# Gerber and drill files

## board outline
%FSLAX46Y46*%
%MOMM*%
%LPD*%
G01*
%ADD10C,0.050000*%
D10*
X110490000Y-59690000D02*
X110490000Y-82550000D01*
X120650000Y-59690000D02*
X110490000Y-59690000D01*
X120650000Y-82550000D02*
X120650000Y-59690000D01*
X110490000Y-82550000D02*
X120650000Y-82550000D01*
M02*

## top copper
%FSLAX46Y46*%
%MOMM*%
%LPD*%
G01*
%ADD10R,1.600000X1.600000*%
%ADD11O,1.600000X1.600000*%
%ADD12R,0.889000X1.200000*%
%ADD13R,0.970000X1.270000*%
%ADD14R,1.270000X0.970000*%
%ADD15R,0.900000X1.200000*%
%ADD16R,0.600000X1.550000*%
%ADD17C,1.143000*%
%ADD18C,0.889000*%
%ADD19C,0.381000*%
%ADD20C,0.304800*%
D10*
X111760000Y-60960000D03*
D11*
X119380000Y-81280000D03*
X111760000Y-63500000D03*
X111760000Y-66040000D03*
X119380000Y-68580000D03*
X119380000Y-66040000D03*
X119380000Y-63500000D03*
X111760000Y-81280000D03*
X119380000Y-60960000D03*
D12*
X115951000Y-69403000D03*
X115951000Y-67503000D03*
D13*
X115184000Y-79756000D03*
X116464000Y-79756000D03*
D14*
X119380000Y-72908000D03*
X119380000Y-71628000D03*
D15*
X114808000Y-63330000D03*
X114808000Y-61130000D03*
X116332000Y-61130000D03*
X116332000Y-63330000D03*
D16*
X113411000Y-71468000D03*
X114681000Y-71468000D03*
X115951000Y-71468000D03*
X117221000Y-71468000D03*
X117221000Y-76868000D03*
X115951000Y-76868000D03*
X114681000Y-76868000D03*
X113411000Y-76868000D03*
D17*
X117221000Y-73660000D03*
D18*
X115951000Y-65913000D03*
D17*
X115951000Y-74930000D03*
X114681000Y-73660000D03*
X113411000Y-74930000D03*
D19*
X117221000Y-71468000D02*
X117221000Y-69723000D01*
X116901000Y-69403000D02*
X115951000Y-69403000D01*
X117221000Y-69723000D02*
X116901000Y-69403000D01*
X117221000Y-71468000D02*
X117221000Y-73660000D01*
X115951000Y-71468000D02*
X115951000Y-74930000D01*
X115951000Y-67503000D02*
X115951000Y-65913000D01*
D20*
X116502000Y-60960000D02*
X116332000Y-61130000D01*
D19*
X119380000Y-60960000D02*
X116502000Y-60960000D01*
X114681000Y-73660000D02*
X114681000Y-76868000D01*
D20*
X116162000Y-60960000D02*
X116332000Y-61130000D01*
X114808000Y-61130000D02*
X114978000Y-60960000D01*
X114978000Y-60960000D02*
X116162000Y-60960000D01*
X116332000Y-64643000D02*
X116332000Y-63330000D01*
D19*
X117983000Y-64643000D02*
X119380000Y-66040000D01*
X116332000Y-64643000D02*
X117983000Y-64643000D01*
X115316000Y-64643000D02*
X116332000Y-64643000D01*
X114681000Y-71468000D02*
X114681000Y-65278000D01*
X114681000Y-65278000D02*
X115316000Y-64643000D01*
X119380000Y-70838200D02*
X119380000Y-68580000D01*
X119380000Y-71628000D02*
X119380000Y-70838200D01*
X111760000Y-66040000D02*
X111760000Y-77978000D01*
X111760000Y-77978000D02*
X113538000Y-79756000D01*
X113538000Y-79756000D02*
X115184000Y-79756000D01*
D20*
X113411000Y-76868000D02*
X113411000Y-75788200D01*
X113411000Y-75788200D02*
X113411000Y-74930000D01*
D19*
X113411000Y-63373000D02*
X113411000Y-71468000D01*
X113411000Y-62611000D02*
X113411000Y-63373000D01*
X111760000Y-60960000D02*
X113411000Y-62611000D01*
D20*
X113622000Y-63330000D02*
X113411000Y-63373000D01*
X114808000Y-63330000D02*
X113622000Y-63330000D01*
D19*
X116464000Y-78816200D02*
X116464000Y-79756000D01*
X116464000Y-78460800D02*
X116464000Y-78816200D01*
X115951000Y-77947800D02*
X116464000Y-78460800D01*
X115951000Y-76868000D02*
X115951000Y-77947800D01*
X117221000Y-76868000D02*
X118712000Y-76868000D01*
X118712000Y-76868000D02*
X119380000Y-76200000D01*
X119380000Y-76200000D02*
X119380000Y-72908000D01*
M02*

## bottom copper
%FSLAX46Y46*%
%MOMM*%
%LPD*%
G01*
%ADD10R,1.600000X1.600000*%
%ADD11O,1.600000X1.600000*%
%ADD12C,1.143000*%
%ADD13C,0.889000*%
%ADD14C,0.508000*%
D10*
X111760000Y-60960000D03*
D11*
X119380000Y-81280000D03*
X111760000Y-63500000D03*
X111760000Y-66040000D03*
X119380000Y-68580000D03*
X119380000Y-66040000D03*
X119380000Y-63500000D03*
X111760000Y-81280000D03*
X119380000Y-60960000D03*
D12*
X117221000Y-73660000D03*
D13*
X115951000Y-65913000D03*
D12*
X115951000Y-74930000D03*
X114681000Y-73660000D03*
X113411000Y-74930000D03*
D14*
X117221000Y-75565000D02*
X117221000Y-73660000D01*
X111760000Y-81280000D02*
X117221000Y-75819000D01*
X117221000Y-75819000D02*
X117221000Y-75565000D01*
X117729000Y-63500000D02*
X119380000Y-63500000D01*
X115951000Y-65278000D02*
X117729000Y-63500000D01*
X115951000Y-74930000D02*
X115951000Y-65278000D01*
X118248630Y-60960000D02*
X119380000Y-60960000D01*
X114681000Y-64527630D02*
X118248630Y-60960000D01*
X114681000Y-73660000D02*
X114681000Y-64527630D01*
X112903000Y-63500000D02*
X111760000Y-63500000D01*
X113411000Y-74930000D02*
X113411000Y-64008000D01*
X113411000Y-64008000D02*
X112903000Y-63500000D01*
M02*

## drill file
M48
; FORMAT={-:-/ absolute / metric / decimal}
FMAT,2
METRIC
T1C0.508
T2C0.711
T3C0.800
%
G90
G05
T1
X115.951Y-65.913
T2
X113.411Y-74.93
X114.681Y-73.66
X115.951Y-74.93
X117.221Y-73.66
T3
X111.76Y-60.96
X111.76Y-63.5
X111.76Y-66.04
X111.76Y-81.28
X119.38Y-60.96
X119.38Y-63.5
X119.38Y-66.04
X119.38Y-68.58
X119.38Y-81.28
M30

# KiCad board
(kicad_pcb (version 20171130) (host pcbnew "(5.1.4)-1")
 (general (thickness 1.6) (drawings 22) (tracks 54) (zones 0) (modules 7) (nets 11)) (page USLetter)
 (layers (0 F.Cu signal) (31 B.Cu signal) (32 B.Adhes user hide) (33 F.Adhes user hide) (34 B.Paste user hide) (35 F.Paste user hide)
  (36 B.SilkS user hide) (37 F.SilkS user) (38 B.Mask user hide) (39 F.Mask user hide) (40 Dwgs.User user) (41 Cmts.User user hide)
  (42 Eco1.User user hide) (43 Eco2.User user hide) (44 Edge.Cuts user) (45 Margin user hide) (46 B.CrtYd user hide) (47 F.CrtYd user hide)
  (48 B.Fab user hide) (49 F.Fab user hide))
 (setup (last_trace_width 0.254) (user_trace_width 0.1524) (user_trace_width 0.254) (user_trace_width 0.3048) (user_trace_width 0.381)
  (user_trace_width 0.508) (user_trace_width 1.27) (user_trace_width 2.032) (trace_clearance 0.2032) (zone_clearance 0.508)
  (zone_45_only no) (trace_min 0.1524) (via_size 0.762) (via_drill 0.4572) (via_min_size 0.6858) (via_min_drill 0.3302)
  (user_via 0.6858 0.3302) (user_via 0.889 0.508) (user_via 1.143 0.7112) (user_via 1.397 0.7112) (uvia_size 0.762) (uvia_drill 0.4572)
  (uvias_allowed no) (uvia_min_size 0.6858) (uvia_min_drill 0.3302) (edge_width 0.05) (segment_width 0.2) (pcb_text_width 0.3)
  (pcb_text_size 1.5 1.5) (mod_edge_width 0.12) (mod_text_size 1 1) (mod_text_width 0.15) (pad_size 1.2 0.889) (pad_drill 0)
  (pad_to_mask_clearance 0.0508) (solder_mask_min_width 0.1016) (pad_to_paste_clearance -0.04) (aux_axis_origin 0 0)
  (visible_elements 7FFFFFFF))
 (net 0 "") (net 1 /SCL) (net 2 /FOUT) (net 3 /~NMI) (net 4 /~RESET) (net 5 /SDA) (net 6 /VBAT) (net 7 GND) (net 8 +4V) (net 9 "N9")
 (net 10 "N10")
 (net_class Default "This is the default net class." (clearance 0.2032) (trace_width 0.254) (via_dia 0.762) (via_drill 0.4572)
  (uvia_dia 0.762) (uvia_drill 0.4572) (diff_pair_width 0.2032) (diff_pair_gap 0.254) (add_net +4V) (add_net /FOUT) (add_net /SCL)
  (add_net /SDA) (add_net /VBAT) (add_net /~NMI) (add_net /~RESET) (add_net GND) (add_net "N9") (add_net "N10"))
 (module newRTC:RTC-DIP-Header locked (layer F.Cu) (at 111.76 60.96)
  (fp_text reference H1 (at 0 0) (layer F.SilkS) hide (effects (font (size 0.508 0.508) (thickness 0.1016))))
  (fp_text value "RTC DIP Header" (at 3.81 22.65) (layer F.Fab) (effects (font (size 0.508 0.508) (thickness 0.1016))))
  (pad 1 thru_hole rect (at 0 0) (size 1.6 1.6) (drill 0.8) (layers *.Cu *.Mask) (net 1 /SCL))
  (pad 10 thru_hole oval (at 7.62 20.32) (size 1.6 1.6) (drill 0.8) (layers *.Cu *.Mask))
  (pad 2 thru_hole oval (at 0 2.54) (size 1.6 1.6) (drill 0.8) (layers *.Cu *.Mask) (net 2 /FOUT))
  (pad 3 thru_hole oval (at 0 5.08) (size 1.6 1.6) (drill 0.8) (layers *.Cu *.Mask) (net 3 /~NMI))
  (pad 15 thru_hole oval (at 7.62 7.62) (size 1.6 1.6) (drill 0.8) (layers *.Cu *.Mask) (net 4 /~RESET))
  (pad 16 thru_hole oval (at 7.62 5.08) (size 1.6 1.6) (drill 0.8) (layers *.Cu *.Mask) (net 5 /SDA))
  (pad 17 thru_hole oval (at 7.62 2.54) (size 1.6 1.6) (drill 0.8) (layers *.Cu *.Mask) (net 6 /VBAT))
  (pad 9 thru_hole oval (at 0 20.32) (size 1.6 1.6) (drill 0.8) (layers *.Cu *.Mask) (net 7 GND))
  (pad 18 thru_hole oval (at 7.62 0) (size 1.6 1.6) (drill 0.8) (layers *.Cu *.Mask) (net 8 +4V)))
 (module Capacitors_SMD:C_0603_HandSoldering (layer F.Cu) (at 115.951 68.453 270)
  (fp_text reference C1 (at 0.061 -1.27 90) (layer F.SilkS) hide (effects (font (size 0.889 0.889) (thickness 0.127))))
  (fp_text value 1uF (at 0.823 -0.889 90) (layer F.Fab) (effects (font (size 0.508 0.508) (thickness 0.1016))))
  (pad 2 smd rect (at 0.95 0 270) (size 1.2 0.889) (layers F.Cu F.Paste F.Mask) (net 7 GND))
  (pad 1 smd rect (at -0.95 0 270) (size 1.2 0.889) (layers F.Cu F.Paste F.Mask) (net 6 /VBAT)))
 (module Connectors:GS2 (layer F.Cu) (at 115.824 79.756 270)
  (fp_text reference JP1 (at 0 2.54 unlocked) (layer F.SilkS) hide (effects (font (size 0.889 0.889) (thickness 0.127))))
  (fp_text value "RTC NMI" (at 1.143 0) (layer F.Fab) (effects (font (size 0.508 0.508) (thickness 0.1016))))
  (pad 2 smd rect (at 0 0.64 270) (size 1.27 0.97) (layers F.Cu F.Paste F.Mask) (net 3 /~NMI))
  (pad 1 smd rect (at 0 -0.64 270) (size 1.27 0.97) (layers F.Cu F.Paste F.Mask) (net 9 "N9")))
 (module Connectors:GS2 (layer F.Cu) (at 119.38 72.268)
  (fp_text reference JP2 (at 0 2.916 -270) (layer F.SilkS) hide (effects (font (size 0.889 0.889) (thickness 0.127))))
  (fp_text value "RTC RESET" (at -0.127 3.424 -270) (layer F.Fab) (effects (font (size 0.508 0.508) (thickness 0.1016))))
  (pad 2 smd rect (at 0 0.64) (size 1.27 0.97) (layers F.Cu F.Paste F.Mask) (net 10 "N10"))
  (pad 1 smd rect (at 0 -0.64) (size 1.27 0.97) (layers F.Cu F.Paste F.Mask) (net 4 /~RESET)))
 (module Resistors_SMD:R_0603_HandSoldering (layer F.Cu) (at 114.808 62.23 270)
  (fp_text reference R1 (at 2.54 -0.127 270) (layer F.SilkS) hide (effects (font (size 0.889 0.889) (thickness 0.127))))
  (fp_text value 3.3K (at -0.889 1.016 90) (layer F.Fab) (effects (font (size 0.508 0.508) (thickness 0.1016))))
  (pad 2 smd rect (at 1.1 0 270) (size 1.2 0.9) (layers F.Cu F.Paste F.Mask) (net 1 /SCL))
  (pad 1 smd rect (at -1.1 0 270) (size 1.2 0.9) (layers F.Cu F.Paste F.Mask) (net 8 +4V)))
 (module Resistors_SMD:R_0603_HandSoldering (layer F.Cu) (at 116.332 62.23 270)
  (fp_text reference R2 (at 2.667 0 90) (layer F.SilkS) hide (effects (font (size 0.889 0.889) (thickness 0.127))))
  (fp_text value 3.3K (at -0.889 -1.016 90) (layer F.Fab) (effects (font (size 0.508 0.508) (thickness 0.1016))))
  (pad 1 smd rect (at -1.1 0 270) (size 1.2 0.9) (layers F.Cu F.Paste F.Mask) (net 8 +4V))
  (pad 2 smd rect (at 1.1 0 270) (size 1.2 0.9) (layers F.Cu F.Paste F.Mask) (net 5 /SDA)))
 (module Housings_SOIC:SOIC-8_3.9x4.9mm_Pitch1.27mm (layer F.Cu) (at 115.316 74.168 90)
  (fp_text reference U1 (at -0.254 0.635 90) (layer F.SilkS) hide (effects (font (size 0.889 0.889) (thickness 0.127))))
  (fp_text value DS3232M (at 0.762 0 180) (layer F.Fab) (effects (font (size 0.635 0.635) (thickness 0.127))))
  (pad 8 smd rect (at 2.7 -1.905 90) (size 1.55 0.6) (layers F.Cu F.Paste F.Mask) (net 1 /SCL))
  (pad 7 smd rect (at 2.7 -0.635 90) (size 1.55 0.6) (layers F.Cu F.Paste F.Mask) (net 5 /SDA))
  (pad 6 smd rect (at 2.7 0.635 90) (size 1.55 0.6) (layers F.Cu F.Paste F.Mask) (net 6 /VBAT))
  (pad 5 smd rect (at 2.7 1.905 90) (size 1.55 0.6) (layers F.Cu F.Paste F.Mask) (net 7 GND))
  (pad 4 smd rect (at -2.7 1.905 90) (size 1.55 0.6) (layers F.Cu F.Paste F.Mask) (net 10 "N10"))
  (pad 3 smd rect (at -2.7 0.635 90) (size 1.55 0.6) (layers F.Cu F.Paste F.Mask) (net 9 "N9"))
  (pad 2 smd rect (at -2.7 -0.635 90) (size 1.55 0.6) (layers F.Cu F.Paste F.Mask) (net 8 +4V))
  (pad 1 smd rect (at -2.7 -1.905 90) (size 1.55 0.6) (layers F.Cu F.Paste F.Mask) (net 2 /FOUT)))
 (gr_line (start 110.49 59.69) (end 110.49 82.55) (layer Edge.Cuts) (width 0.05))
 (gr_line (start 120.65 59.69) (end 110.49 59.69) (layer Edge.Cuts) (width 0.05))
 (gr_line (start 120.65 82.55) (end 120.65 59.69) (layer Edge.Cuts) (width 0.05))
 (gr_line (start 110.49 82.55) (end 120.65 82.55) (layer Edge.Cuts) (width 0.05))
 (via (at 117.221 73.66) (size 1.143) (drill 0.7112) (layers F.Cu B.Cu) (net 7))
 (segment (start 117.221 71.468) (end 117.221 69.723) (width 0.381) (layer F.Cu) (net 7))
 (segment (start 116.901 69.403) (end 115.951 69.403) (width 0.381) (layer F.Cu) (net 7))
 (segment (start 117.221 69.723) (end 116.901 69.403) (width 0.381) (layer F.Cu) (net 7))
 (segment (start 117.221 75.565) (end 117.221 73.66) (width 0.508) (layer B.Cu) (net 7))
 (segment (start 111.76 81.28) (end 117.221 75.819) (width 0.508) (layer B.Cu) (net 7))
 (segment (start 117.221 75.819) (end 117.221 75.565) (width 0.508) (layer B.Cu) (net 7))
 (segment (start 117.221 71.468) (end 117.221 73.66) (width 0.381) (layer F.Cu) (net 7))
 (via (at 115.951 65.913) (size 0.889) (drill 0.508) (layers F.Cu B.Cu) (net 6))
 (via (at 115.951 74.93) (size 1.143) (drill 0.7112) (layers F.Cu B.Cu) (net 6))
 (segment (start 117.729 63.5) (end 119.38 63.5) (width 0.508) (layer B.Cu) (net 6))
 (segment (start 115.951 65.278) (end 117.729 63.5) (width 0.508) (layer B.Cu) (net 6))
 (segment (start 115.951 71.468) (end 115.951 74.93) (width 0.381) (layer F.Cu) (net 6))
 (segment (start 115.951 74.93) (end 115.951 65.278) (width 0.508) (layer B.Cu) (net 6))
 (segment (start 115.951 67.503) (end 115.951 65.913) (width 0.381) (layer F.Cu) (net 6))
 (segment (start 116.502 60.96) (end 116.332 61.13) (width 0.3048) (layer F.Cu) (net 8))
 (segment (start 119.38 60.96) (end 116.502 60.96) (width 0.381) (layer F.Cu) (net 8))
 (via (at 114.681 73.66) (size 1.143) (drill 0.7112) (layers F.Cu B.Cu) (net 8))
 (segment (start 114.681 73.66) (end 114.681 76.868) (width 0.381) (layer F.Cu) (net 8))
 (segment (start 118.24863 60.96) (end 119.38 60.96) (width 0.508) (layer B.Cu) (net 8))
 (segment (start 114.681 64.52763) (end 118.24863 60.96) (width 0.508) (layer B.Cu) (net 8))
 (segment (start 114.681 73.66) (end 114.681 64.52763) (width 0.508) (layer B.Cu) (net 8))
 (segment (start 116.162 60.96) (end 116.332 61.13) (width 0.3048) (layer F.Cu) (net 8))
 (segment (start 114.808 61.13) (end 114.978 60.96) (width 0.3048) (layer F.Cu) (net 8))
 (segment (start 114.978 60.96) (end 116.162 60.96) (width 0.3048) (layer F.Cu) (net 8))
 (segment (start 116.332 64.643) (end 116.332 63.33) (width 0.3048) (layer F.Cu) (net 5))
 (segment (start 117.983 64.643) (end 119.38 66.04) (width 0.381) (layer F.Cu) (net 5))
 (segment (start 116.332 64.643) (end 117.983 64.643) (width 0.381) (layer F.Cu) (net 5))
 (segment (start 115.316 64.643) (end 116.332 64.643) (width 0.381) (layer F.Cu) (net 5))
 (segment (start 114.681 71.468) (end 114.681 65.278) (width 0.381) (layer F.Cu) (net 5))
 (segment (start 114.681 65.278) (end 115.316 64.643) (width 0.381) (layer F.Cu) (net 5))
 (segment (start 119.38 70.8382) (end 119.38 68.58) (width 0.381) (layer F.Cu) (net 4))
 (segment (start 119.38 71.628) (end 119.38 70.8382) (width 0.381) (layer F.Cu) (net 4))
 (segment (start 111.76 66.04) (end 111.76 77.978) (width 0.381) (layer F.Cu) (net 3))
 (segment (start 111.76 77.978) (end 113.538 79.756) (width 0.381) (layer F.Cu) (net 3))
 (segment (start 113.538 79.756) (end 115.184 79.756) (width 0.381) (layer F.Cu) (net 3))
 (segment (start 113.411 76.868) (end 113.411 75.7882) (width 0.3048) (layer F.Cu) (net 2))
 (segment (start 113.411 75.7882) (end 113.411 74.93) (width 0.3048) (layer F.Cu) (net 2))
 (via (at 113.411 74.93) (size 1.143) (drill 0.7112) (layers F.Cu B.Cu) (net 2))
 (segment (start 112.903 63.5) (end 111.76 63.5) (width 0.508) (layer B.Cu) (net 2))
 (segment (start 113.411 74.93) (end 113.411 64.008) (width 0.508) (layer B.Cu) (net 2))
 (segment (start 113.411 64.008) (end 112.903 63.5) (width 0.508) (layer B.Cu) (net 2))
 (segment (start 113.411 63.373) (end 113.411 71.468) (width 0.381) (layer F.Cu) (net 1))
 (segment (start 113.411 62.611) (end 113.411 63.373) (width 0.381) (layer F.Cu) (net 1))
 (segment (start 111.76 60.96) (end 113.411 62.611) (width 0.381) (layer F.Cu) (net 1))
 (segment (start 113.622 63.33) (end 113.411 63.373) (width 0.3048) (layer F.Cu) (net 1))
 (segment (start 114.808 63.33) (end 113.622 63.33) (width 0.3048) (layer F.Cu) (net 1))
 (segment (start 116.464 78.8162) (end 116.464 79.756) (width 0.381) (layer F.Cu) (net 9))
 (segment (start 116.464 78.4608) (end 116.464 78.8162) (width 0.381) (layer F.Cu) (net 9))
 (segment (start 115.951 77.9478) (end 116.464 78.4608) (width 0.381) (layer F.Cu) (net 9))
 (segment (start 115.951 76.868) (end 115.951 77.9478) (width 0.381) (layer F.Cu) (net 9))
 (segment (start 117.221 76.868) (end 118.712 76.868) (width 0.381) (layer F.Cu) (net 10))
 (segment (start 118.712 76.868) (end 119.38 76.2) (width 0.381) (layer F.Cu) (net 10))
 (segment (start 119.38 76.2) (end 119.38 72.908) (width 0.381) (layer F.Cu) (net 10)))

